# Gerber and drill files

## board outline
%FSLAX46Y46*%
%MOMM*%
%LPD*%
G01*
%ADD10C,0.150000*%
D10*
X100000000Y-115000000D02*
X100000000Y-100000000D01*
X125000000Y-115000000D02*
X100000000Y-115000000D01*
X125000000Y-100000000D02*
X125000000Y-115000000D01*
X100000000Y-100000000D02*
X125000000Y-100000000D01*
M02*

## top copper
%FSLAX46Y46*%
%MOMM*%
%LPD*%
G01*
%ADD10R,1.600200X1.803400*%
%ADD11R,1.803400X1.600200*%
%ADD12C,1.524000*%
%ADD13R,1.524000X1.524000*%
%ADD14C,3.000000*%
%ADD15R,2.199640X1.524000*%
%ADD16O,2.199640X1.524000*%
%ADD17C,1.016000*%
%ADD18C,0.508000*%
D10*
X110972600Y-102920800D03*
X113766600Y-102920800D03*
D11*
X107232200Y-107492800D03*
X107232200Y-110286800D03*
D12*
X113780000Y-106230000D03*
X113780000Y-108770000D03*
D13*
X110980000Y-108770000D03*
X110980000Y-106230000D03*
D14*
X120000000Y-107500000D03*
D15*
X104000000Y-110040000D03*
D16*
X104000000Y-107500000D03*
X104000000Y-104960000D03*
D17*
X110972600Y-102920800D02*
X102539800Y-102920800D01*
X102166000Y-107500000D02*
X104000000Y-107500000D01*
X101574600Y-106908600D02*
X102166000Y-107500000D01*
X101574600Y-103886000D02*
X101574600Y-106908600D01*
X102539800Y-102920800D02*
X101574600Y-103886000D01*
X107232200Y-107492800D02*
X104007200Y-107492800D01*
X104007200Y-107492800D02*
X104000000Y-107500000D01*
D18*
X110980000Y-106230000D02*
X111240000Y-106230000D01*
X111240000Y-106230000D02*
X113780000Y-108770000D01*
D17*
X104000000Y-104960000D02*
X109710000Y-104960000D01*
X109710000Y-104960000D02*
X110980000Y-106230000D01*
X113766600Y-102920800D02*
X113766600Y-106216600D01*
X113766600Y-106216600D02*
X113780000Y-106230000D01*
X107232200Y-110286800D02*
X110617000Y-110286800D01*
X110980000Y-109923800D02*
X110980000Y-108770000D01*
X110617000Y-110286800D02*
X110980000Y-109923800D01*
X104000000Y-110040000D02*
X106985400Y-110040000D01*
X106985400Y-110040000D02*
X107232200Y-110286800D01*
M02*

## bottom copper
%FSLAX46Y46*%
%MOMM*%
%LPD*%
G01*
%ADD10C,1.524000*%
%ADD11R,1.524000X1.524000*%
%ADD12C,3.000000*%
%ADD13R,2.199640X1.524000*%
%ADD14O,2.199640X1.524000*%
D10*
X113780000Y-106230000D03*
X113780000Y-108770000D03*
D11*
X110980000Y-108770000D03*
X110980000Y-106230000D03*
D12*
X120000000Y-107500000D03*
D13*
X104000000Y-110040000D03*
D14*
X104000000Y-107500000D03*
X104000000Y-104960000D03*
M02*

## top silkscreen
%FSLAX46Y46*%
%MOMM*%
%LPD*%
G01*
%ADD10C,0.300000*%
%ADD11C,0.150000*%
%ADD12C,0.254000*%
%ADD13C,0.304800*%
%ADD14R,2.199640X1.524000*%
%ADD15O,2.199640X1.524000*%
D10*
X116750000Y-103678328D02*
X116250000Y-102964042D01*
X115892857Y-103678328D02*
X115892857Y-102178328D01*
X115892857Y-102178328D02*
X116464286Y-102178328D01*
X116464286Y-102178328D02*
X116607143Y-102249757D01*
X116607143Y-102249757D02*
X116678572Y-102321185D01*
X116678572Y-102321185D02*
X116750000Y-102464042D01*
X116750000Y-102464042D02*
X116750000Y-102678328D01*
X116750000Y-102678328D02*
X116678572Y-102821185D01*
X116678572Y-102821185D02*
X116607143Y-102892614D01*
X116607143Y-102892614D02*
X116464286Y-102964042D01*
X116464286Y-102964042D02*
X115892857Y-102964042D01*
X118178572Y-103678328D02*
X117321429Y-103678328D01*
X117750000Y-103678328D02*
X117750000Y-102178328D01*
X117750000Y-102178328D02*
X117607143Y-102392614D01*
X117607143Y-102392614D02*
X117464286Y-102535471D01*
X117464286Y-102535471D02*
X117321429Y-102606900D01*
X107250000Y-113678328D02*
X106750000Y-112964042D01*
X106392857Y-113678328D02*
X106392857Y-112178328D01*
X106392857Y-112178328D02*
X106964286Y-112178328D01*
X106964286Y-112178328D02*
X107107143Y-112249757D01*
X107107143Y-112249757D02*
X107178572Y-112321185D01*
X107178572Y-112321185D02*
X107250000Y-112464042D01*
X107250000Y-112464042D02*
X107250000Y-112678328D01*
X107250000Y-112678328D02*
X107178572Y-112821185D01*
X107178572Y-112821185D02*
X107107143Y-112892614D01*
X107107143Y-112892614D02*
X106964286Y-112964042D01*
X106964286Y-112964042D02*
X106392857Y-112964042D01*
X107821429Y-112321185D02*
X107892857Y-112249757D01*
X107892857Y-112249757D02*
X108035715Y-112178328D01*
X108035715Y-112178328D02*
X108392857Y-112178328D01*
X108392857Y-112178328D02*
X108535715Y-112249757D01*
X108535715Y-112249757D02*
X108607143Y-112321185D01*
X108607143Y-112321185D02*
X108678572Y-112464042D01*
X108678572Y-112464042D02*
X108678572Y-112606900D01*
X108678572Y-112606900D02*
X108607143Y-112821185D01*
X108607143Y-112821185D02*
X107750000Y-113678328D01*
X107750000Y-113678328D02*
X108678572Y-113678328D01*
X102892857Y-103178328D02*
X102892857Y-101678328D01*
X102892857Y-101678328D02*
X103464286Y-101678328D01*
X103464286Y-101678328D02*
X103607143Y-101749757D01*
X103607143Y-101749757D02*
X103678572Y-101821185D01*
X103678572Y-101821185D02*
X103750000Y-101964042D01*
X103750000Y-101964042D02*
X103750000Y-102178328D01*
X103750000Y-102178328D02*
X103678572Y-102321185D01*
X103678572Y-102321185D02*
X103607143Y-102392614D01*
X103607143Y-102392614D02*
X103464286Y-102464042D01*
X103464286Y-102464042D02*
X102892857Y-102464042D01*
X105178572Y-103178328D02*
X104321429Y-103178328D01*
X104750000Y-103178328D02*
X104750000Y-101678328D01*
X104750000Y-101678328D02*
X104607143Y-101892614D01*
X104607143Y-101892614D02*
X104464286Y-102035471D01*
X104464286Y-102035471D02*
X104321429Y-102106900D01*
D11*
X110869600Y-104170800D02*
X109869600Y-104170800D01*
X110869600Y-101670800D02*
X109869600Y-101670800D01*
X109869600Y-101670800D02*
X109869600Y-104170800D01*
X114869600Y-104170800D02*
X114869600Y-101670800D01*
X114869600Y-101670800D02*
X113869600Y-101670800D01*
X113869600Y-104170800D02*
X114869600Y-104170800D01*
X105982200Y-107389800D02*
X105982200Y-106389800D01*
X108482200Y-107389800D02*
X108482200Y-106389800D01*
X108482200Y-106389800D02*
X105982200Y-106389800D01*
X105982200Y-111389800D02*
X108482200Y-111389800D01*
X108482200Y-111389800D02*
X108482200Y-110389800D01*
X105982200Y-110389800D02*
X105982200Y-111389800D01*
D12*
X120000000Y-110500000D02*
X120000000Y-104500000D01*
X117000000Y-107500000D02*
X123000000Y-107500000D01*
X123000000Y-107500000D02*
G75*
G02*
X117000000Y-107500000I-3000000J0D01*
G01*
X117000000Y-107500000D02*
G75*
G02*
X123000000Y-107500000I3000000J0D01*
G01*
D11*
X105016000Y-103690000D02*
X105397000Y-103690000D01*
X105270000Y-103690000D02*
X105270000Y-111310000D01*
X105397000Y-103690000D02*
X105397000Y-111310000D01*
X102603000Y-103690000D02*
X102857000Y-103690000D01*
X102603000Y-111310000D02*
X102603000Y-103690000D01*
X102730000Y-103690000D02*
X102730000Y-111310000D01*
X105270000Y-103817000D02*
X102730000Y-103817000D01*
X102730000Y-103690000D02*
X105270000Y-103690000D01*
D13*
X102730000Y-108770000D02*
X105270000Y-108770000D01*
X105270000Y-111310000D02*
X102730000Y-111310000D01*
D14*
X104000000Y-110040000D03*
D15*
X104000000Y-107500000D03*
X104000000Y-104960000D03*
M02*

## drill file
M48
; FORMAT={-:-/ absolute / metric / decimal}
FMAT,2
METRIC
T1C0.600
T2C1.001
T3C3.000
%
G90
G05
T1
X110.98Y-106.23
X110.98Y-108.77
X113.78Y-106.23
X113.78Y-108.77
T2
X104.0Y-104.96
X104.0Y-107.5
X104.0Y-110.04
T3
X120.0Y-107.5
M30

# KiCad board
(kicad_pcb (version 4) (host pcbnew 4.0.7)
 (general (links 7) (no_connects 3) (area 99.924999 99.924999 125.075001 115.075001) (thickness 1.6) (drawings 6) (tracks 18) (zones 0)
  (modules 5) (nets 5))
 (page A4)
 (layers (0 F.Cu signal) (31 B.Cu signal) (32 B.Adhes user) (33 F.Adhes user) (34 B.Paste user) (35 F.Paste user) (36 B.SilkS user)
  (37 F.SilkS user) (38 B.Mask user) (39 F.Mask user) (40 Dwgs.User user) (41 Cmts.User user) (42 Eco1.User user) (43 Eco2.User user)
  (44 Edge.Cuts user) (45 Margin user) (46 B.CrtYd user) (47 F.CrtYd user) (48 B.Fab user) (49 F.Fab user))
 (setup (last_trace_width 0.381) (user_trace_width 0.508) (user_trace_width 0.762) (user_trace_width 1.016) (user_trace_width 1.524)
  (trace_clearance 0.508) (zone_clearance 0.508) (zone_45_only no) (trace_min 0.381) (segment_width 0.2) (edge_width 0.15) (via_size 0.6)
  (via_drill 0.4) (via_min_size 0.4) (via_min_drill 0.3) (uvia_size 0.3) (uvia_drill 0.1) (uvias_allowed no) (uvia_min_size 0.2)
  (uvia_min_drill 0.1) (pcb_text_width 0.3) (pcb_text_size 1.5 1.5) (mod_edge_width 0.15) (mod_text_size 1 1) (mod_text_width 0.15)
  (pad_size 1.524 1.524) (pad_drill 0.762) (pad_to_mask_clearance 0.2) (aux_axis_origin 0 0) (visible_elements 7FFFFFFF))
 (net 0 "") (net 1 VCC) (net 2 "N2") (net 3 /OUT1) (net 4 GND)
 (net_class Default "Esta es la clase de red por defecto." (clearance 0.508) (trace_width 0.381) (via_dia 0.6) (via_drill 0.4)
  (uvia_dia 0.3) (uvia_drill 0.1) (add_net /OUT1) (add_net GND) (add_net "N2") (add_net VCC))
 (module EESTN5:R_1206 (layer F.Cu) (at 112.3696 102.9208 180)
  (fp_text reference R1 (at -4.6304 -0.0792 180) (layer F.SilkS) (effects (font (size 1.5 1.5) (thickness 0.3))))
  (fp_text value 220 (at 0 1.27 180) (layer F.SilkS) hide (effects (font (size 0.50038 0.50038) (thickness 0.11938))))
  (fp_line (start 1.5 -1.25) (end 2.5 -1.25) (layer F.SilkS) (width 0.15))
  (fp_line (start 1.5 1.25) (end 2.5 1.25) (layer F.SilkS) (width 0.15))
  (fp_line (start 2.5 1.25) (end 2.5 -1.25) (layer F.SilkS) (width 0.15))
  (fp_line (start -2.5 -1.25) (end -2.5 1.25) (layer F.SilkS) (width 0.15))
  (fp_line (start -2.5 1.25) (end -1.5 1.25) (layer F.SilkS) (width 0.15))
  (fp_line (start -1.5 -1.25) (end -2.5 -1.25) (layer F.SilkS) (width 0.15))
  (pad 1 smd rect (at 1.397 0 180) (size 1.6002 1.8034) (layers F.Cu F.Paste F.Mask) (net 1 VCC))
  (pad 2 smd rect (at -1.397 0 180) (size 1.6002 1.8034) (layers F.Cu F.Paste F.Mask) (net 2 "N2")))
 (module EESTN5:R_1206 (layer F.Cu) (at 107.2322 108.8898 90)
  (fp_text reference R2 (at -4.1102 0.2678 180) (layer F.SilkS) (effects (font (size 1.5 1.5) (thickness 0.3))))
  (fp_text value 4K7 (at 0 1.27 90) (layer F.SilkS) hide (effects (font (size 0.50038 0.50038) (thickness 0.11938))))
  (fp_line (start 1.5 -1.25) (end 2.5 -1.25) (layer F.SilkS) (width 0.15))
  (fp_line (start 1.5 1.25) (end 2.5 1.25) (layer F.SilkS) (width 0.15))
  (fp_line (start 2.5 1.25) (end 2.5 -1.25) (layer F.SilkS) (width 0.15))
  (fp_line (start -2.5 -1.25) (end -2.5 1.25) (layer F.SilkS) (width 0.15))
  (fp_line (start -2.5 1.25) (end -1.5 1.25) (layer F.SilkS) (width 0.15))
  (fp_line (start -1.5 -1.25) (end -2.5 -1.25) (layer F.SilkS) (width 0.15))
  (pad 1 smd rect (at 1.397 0 90) (size 1.6002 1.8034) (layers F.Cu F.Paste F.Mask) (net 1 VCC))
  (pad 2 smd rect (at -1.397 0 90) (size 1.6002 1.8034) (layers F.Cu F.Paste F.Mask) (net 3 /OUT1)))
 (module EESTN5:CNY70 (layer B.Cu) (at 112.38 107.5 180)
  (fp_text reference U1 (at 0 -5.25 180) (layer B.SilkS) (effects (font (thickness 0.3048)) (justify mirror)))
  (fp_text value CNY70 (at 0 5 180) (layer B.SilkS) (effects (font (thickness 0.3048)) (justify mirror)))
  (pad 1 thru_hole circle (at -1.4 1.27 180) (size 1.524 1.524) (drill 0.6) (layers *.Cu *.Mask B.SilkS) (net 2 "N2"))
  (pad 2 thru_hole circle (at -1.4 -1.27 180) (size 1.524 1.524) (drill 0.6) (layers *.Cu *.Mask B.SilkS) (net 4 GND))
  (pad 3 thru_hole rect (at 1.4 -1.27 180) (size 1.524 1.524) (drill 0.6) (layers *.Cu *.Mask B.SilkS) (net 3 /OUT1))
  (pad 4 thru_hole rect (at 1.4 1.27 180) (size 1.524 1.524) (drill 0.6) (layers *.Cu *.Mask B.SilkS) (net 4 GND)))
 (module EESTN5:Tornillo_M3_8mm (layer B.Cu) (at 120 107.5)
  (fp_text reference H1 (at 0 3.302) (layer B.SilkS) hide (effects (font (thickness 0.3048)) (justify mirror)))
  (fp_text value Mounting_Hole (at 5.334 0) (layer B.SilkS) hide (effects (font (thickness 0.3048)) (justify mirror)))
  (fp_line (start 0 3) (end 0 -3) (layer F.SilkS) (width 0.254))
  (fp_line (start -3 0) (end 3 0) (layer F.SilkS) (width 0.254))
  (fp_circle (center 0 0) (end 3 0) (layer F.SilkS) (width 0.254))
  (pad 1 thru_hole circle (at 0 0) (size 3 3) (drill 3) (layers *.Cu B.SilkS)))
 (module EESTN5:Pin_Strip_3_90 (layer F.Cu) (at 104 107.5 90)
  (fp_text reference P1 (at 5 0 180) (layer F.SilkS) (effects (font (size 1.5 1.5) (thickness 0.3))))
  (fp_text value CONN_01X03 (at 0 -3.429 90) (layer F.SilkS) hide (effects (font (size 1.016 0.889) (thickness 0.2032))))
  (fp_line (start 3.81 1.016) (end 3.81 1.397) (layer F.SilkS) (width 0.15))
  (fp_line (start 3.81 1.27) (end -3.81 1.27) (layer F.SilkS) (width 0.15))
  (fp_line (start 3.81 1.397) (end -3.81 1.397) (layer F.SilkS) (width 0.15))
  (fp_line (start 3.81 -1.397) (end 3.81 -1.143) (layer F.SilkS) (width 0.15))
  (fp_line (start -3.81 -1.397) (end 3.81 -1.397) (layer F.SilkS) (width 0.15))
  (fp_line (start 3.81 -1.27) (end -3.81 -1.27) (layer F.SilkS) (width 0.15))
  (fp_line (start 3.683 1.27) (end 3.683 -1.27) (layer F.SilkS) (width 0.15))
  (fp_line (start 3.81 -1.27) (end 3.81 1.27) (layer F.SilkS) (width 0.15))
  (fp_line (start -1.27 -1.27) (end -1.27 1.27) (layer F.SilkS) (width 0.3048))
  (fp_line (start -3.81 1.27) (end -3.81 -1.27) (layer F.SilkS) (width 0.3048))
  (pad 1 thru_hole rect (at -2.54 0 90) (size 1.524 2.19964) (drill 1.00076) (layers *.Cu *.Mask F.SilkS) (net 3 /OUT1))
  (pad 2 thru_hole oval (at 0 0 90) (size 1.524 2.19964) (drill 1.00076) (layers *.Cu *.Mask F.SilkS) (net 1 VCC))
  (pad 3 thru_hole oval (at 2.54 0 90) (size 1.524 2.19964) (drill 1.00076) (layers *.Cu *.Mask F.SilkS) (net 4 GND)))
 (gr_line (start 100 115) (end 100 100) (layer Edge.Cuts) (width 0.15))
 (gr_line (start 125 115) (end 100 115) (layer Edge.Cuts) (width 0.15))
 (gr_line (start 125 100) (end 125 115) (layer Edge.Cuts) (width 0.15))
 (gr_line (start 100 100) (end 125 100) (layer Edge.Cuts) (width 0.15))
 (segment (start 110.9726 102.9208) (end 102.5398 102.9208) (width 1.016) (layer F.Cu) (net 1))
 (segment (start 102.166 107.5) (end 104 107.5) (width 1.016) (layer F.Cu) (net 1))
 (segment (start 101.5746 106.9086) (end 102.166 107.5) (width 1.016) (layer F.Cu) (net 1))
 (segment (start 101.5746 103.886) (end 101.5746 106.9086) (width 1.016) (layer F.Cu) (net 1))
 (segment (start 102.5398 102.9208) (end 101.5746 103.886) (width 1.016) (layer F.Cu) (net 1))
 (segment (start 107.2322 107.4928) (end 104.0072 107.4928) (width 1.016) (layer F.Cu) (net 1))
 (segment (start 104.0072 107.4928) (end 104 107.5) (width 1.016) (layer F.Cu) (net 1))
 (segment (start 110.98 106.23) (end 111.24 106.23) (width 0.508) (layer F.Cu) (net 4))
 (segment (start 111.24 106.23) (end 113.78 108.77) (width 0.508) (layer F.Cu) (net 4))
 (segment (start 104 104.96) (end 109.71 104.96) (width 1.016) (layer F.Cu) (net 4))
 (segment (start 109.71 104.96) (end 110.98 106.23) (width 1.016) (layer F.Cu) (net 4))
 (segment (start 113.7666 102.9208) (end 113.7666 106.2166) (width 1.016) (layer F.Cu) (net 2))
 (segment (start 113.7666 106.2166) (end 113.78 106.23) (width 1.016) (layer F.Cu) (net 2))
 (segment (start 107.2322 110.2868) (end 110.617 110.2868) (width 1.016) (layer F.Cu) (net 3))
 (segment (start 110.98 109.9238) (end 110.98 108.77) (width 1.016) (layer F.Cu) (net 3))
 (segment (start 110.617 110.2868) (end 110.98 109.9238) (width 1.016) (layer F.Cu) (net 3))
 (segment (start 104 110.04) (end 106.9854 110.04) (width 1.016) (layer F.Cu) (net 3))
 (segment (start 106.9854 110.04) (end 107.2322 110.2868) (width 1.016) (layer F.Cu) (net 3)))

